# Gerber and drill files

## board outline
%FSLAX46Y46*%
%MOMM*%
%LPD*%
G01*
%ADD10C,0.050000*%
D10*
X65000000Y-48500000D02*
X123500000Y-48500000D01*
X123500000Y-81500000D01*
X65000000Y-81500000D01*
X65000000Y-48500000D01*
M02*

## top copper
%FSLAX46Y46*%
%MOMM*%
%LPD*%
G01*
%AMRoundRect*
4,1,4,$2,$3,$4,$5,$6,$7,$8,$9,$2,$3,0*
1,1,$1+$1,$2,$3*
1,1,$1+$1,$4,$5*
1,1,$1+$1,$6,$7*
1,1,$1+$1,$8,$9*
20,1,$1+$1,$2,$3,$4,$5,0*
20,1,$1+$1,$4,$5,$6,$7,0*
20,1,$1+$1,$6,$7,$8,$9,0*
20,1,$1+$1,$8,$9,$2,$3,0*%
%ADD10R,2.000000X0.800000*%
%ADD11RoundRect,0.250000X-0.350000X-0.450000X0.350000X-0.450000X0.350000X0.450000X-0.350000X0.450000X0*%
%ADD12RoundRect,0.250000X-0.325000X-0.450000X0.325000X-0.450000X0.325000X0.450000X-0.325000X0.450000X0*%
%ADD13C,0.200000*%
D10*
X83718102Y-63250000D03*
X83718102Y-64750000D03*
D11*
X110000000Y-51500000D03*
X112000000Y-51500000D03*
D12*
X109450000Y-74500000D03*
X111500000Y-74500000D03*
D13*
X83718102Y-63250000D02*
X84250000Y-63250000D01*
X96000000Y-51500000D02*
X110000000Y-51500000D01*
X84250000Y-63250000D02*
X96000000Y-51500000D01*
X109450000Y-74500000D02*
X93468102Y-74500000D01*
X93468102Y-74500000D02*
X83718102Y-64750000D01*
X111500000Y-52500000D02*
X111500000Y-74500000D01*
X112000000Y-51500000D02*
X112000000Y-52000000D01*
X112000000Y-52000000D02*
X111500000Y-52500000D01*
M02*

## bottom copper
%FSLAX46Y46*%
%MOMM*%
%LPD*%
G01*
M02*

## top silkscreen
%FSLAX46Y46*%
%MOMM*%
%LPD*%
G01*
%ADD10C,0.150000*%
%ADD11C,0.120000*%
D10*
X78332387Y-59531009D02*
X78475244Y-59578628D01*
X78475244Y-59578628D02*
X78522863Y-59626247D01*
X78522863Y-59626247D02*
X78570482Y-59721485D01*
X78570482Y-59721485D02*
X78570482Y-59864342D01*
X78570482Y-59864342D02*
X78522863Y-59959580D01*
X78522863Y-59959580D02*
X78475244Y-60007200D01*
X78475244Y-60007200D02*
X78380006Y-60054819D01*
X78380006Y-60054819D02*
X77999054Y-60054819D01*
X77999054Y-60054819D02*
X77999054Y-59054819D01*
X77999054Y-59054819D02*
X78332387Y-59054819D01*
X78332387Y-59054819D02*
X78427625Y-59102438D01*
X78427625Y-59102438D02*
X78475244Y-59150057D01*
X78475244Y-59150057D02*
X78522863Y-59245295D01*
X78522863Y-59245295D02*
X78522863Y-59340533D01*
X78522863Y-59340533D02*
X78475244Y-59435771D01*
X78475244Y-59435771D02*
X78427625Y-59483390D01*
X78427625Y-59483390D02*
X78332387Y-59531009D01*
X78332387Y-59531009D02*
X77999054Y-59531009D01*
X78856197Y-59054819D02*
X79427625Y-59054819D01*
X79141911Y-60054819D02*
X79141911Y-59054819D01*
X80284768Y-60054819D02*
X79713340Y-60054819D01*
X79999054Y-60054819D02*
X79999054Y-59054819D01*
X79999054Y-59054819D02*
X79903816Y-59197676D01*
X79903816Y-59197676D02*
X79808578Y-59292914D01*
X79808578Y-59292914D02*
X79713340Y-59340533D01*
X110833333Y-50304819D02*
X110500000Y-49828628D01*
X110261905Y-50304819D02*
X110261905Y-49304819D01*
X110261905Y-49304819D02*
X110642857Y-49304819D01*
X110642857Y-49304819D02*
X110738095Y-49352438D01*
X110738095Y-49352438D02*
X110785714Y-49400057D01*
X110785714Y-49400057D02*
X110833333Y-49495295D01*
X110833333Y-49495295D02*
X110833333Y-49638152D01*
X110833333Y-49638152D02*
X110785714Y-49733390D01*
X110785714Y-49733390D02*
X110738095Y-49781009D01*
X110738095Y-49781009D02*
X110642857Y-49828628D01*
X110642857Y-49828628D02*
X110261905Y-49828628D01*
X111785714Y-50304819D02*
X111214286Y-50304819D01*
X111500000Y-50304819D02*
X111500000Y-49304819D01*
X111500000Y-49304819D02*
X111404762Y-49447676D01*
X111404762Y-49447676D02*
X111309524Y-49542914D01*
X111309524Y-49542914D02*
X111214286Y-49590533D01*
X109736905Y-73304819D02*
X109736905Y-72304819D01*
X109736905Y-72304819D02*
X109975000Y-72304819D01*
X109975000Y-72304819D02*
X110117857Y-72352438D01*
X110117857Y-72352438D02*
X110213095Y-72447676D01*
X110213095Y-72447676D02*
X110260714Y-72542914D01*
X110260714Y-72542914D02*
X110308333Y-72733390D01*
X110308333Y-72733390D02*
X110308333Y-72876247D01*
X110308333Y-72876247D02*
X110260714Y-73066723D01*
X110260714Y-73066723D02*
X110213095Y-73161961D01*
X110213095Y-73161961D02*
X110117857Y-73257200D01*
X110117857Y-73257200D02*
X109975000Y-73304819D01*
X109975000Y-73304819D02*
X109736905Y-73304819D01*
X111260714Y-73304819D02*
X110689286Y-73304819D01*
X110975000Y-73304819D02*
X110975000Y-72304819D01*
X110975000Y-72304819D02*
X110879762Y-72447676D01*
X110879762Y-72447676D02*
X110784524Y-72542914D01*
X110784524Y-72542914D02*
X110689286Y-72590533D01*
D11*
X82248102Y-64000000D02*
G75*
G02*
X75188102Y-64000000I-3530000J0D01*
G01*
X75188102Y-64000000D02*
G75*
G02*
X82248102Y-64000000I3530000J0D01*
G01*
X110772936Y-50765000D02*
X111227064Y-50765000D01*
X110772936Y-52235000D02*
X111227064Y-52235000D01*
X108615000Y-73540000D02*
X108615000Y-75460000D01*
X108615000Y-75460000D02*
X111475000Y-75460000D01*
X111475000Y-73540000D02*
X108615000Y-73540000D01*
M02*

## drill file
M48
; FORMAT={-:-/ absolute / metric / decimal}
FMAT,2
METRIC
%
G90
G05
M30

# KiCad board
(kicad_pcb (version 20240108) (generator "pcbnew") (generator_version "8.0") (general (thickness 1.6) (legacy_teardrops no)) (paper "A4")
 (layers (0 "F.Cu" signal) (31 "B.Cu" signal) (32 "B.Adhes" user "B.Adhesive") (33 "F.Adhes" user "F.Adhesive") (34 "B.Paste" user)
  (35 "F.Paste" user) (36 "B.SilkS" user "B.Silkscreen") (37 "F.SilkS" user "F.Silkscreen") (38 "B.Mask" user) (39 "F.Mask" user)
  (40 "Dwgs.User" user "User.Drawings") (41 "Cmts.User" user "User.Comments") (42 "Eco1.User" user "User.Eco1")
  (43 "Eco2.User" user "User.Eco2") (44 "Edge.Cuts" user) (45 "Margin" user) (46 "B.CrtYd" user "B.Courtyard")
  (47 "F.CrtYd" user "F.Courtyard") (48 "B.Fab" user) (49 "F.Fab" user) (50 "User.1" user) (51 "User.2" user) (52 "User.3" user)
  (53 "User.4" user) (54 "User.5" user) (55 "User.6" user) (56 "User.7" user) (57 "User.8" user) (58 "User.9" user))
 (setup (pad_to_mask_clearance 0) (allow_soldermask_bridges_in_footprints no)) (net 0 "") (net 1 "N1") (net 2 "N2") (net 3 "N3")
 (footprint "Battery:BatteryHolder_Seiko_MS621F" (layer "F.Cu") (at 83.718102 64)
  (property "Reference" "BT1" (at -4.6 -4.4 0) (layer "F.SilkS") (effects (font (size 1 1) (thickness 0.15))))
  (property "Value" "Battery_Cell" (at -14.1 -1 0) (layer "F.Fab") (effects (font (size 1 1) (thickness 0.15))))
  (fp_circle (center -5 0) (end -1.47 0) (stroke (width 0.12) (type solid)) (fill none) (layer "F.SilkS"))
  (pad "1" smd rect (at 0 -0.75) (size 2 0.8) (layers "F.Cu" "F.Paste" "F.Mask") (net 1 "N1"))
  (pad "2" smd rect (at 0 0.75) (size 2 0.8) (layers "F.Cu" "F.Paste" "F.Mask") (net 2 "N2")))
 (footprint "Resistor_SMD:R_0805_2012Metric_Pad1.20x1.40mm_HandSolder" (layer "F.Cu") (at 111 51.5)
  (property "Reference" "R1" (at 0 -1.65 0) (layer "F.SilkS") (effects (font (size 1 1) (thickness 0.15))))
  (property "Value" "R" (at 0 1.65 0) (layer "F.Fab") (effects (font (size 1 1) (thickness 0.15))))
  (fp_line (start -0.227064 -0.735) (end 0.227064 -0.735) (stroke (width 0.12) (type solid)) (layer "F.SilkS"))
  (fp_line (start -0.227064 0.735) (end 0.227064 0.735) (stroke (width 0.12) (type solid)) (layer "F.SilkS"))
  (pad "1" smd roundrect (at -1 0) (size 1.2 1.4) (layers "F.Cu" "F.Paste" "F.Mask") (roundrect_rratio 0.208333) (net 1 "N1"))
  (pad "2" smd roundrect (at 1 0) (size 1.2 1.4) (layers "F.Cu" "F.Paste" "F.Mask") (roundrect_rratio 0.208333) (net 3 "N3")))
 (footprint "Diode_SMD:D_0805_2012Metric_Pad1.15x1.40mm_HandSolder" (layer "F.Cu") (at 110.475 74.5)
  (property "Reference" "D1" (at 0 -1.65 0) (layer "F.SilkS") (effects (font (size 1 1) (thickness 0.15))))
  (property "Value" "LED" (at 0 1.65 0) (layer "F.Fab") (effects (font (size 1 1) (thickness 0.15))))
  (fp_line (start -1.86 -0.96) (end -1.86 0.96) (stroke (width 0.12) (type solid)) (layer "F.SilkS"))
  (fp_line (start -1.86 0.96) (end 1 0.96) (stroke (width 0.12) (type solid)) (layer "F.SilkS"))
  (fp_line (start 1 -0.96) (end -1.86 -0.96) (stroke (width 0.12) (type solid)) (layer "F.SilkS"))
  (pad "1" smd roundrect (at -1.025 0) (size 1.15 1.4) (layers "F.Cu" "F.Paste" "F.Mask") (roundrect_rratio 0.217391) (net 2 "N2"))
  (pad "2" smd roundrect (at 1.025 0) (size 1.15 1.4) (layers "F.Cu" "F.Paste" "F.Mask") (roundrect_rratio 0.217391) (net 3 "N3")))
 (gr_rect (start 65 48.5) (end 123.5 81.5) (stroke (width 0.05) (type default)) (fill none) (layer "Edge.Cuts"))
 (segment (start 83.718102 63.25) (end 84.25 63.25) (width 0.2) (layer "F.Cu") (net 1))
 (segment (start 96 51.5) (end 110 51.5) (width 0.2) (layer "F.Cu") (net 1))
 (segment (start 84.25 63.25) (end 96 51.5) (width 0.2) (layer "F.Cu") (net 1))
 (segment (start 109.45 74.5) (end 93.468102 74.5) (width 0.2) (layer "F.Cu") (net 2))
 (segment (start 93.468102 74.5) (end 83.718102 64.75) (width 0.2) (layer "F.Cu") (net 2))
 (segment (start 111.5 52.5) (end 111.5 74.5) (width 0.2) (layer "F.Cu") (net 3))
 (segment (start 112 51.5) (end 112 52) (width 0.2) (layer "F.Cu") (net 3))
 (segment (start 112 52) (end 111.5 52.5) (width 0.2) (layer "F.Cu") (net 3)))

